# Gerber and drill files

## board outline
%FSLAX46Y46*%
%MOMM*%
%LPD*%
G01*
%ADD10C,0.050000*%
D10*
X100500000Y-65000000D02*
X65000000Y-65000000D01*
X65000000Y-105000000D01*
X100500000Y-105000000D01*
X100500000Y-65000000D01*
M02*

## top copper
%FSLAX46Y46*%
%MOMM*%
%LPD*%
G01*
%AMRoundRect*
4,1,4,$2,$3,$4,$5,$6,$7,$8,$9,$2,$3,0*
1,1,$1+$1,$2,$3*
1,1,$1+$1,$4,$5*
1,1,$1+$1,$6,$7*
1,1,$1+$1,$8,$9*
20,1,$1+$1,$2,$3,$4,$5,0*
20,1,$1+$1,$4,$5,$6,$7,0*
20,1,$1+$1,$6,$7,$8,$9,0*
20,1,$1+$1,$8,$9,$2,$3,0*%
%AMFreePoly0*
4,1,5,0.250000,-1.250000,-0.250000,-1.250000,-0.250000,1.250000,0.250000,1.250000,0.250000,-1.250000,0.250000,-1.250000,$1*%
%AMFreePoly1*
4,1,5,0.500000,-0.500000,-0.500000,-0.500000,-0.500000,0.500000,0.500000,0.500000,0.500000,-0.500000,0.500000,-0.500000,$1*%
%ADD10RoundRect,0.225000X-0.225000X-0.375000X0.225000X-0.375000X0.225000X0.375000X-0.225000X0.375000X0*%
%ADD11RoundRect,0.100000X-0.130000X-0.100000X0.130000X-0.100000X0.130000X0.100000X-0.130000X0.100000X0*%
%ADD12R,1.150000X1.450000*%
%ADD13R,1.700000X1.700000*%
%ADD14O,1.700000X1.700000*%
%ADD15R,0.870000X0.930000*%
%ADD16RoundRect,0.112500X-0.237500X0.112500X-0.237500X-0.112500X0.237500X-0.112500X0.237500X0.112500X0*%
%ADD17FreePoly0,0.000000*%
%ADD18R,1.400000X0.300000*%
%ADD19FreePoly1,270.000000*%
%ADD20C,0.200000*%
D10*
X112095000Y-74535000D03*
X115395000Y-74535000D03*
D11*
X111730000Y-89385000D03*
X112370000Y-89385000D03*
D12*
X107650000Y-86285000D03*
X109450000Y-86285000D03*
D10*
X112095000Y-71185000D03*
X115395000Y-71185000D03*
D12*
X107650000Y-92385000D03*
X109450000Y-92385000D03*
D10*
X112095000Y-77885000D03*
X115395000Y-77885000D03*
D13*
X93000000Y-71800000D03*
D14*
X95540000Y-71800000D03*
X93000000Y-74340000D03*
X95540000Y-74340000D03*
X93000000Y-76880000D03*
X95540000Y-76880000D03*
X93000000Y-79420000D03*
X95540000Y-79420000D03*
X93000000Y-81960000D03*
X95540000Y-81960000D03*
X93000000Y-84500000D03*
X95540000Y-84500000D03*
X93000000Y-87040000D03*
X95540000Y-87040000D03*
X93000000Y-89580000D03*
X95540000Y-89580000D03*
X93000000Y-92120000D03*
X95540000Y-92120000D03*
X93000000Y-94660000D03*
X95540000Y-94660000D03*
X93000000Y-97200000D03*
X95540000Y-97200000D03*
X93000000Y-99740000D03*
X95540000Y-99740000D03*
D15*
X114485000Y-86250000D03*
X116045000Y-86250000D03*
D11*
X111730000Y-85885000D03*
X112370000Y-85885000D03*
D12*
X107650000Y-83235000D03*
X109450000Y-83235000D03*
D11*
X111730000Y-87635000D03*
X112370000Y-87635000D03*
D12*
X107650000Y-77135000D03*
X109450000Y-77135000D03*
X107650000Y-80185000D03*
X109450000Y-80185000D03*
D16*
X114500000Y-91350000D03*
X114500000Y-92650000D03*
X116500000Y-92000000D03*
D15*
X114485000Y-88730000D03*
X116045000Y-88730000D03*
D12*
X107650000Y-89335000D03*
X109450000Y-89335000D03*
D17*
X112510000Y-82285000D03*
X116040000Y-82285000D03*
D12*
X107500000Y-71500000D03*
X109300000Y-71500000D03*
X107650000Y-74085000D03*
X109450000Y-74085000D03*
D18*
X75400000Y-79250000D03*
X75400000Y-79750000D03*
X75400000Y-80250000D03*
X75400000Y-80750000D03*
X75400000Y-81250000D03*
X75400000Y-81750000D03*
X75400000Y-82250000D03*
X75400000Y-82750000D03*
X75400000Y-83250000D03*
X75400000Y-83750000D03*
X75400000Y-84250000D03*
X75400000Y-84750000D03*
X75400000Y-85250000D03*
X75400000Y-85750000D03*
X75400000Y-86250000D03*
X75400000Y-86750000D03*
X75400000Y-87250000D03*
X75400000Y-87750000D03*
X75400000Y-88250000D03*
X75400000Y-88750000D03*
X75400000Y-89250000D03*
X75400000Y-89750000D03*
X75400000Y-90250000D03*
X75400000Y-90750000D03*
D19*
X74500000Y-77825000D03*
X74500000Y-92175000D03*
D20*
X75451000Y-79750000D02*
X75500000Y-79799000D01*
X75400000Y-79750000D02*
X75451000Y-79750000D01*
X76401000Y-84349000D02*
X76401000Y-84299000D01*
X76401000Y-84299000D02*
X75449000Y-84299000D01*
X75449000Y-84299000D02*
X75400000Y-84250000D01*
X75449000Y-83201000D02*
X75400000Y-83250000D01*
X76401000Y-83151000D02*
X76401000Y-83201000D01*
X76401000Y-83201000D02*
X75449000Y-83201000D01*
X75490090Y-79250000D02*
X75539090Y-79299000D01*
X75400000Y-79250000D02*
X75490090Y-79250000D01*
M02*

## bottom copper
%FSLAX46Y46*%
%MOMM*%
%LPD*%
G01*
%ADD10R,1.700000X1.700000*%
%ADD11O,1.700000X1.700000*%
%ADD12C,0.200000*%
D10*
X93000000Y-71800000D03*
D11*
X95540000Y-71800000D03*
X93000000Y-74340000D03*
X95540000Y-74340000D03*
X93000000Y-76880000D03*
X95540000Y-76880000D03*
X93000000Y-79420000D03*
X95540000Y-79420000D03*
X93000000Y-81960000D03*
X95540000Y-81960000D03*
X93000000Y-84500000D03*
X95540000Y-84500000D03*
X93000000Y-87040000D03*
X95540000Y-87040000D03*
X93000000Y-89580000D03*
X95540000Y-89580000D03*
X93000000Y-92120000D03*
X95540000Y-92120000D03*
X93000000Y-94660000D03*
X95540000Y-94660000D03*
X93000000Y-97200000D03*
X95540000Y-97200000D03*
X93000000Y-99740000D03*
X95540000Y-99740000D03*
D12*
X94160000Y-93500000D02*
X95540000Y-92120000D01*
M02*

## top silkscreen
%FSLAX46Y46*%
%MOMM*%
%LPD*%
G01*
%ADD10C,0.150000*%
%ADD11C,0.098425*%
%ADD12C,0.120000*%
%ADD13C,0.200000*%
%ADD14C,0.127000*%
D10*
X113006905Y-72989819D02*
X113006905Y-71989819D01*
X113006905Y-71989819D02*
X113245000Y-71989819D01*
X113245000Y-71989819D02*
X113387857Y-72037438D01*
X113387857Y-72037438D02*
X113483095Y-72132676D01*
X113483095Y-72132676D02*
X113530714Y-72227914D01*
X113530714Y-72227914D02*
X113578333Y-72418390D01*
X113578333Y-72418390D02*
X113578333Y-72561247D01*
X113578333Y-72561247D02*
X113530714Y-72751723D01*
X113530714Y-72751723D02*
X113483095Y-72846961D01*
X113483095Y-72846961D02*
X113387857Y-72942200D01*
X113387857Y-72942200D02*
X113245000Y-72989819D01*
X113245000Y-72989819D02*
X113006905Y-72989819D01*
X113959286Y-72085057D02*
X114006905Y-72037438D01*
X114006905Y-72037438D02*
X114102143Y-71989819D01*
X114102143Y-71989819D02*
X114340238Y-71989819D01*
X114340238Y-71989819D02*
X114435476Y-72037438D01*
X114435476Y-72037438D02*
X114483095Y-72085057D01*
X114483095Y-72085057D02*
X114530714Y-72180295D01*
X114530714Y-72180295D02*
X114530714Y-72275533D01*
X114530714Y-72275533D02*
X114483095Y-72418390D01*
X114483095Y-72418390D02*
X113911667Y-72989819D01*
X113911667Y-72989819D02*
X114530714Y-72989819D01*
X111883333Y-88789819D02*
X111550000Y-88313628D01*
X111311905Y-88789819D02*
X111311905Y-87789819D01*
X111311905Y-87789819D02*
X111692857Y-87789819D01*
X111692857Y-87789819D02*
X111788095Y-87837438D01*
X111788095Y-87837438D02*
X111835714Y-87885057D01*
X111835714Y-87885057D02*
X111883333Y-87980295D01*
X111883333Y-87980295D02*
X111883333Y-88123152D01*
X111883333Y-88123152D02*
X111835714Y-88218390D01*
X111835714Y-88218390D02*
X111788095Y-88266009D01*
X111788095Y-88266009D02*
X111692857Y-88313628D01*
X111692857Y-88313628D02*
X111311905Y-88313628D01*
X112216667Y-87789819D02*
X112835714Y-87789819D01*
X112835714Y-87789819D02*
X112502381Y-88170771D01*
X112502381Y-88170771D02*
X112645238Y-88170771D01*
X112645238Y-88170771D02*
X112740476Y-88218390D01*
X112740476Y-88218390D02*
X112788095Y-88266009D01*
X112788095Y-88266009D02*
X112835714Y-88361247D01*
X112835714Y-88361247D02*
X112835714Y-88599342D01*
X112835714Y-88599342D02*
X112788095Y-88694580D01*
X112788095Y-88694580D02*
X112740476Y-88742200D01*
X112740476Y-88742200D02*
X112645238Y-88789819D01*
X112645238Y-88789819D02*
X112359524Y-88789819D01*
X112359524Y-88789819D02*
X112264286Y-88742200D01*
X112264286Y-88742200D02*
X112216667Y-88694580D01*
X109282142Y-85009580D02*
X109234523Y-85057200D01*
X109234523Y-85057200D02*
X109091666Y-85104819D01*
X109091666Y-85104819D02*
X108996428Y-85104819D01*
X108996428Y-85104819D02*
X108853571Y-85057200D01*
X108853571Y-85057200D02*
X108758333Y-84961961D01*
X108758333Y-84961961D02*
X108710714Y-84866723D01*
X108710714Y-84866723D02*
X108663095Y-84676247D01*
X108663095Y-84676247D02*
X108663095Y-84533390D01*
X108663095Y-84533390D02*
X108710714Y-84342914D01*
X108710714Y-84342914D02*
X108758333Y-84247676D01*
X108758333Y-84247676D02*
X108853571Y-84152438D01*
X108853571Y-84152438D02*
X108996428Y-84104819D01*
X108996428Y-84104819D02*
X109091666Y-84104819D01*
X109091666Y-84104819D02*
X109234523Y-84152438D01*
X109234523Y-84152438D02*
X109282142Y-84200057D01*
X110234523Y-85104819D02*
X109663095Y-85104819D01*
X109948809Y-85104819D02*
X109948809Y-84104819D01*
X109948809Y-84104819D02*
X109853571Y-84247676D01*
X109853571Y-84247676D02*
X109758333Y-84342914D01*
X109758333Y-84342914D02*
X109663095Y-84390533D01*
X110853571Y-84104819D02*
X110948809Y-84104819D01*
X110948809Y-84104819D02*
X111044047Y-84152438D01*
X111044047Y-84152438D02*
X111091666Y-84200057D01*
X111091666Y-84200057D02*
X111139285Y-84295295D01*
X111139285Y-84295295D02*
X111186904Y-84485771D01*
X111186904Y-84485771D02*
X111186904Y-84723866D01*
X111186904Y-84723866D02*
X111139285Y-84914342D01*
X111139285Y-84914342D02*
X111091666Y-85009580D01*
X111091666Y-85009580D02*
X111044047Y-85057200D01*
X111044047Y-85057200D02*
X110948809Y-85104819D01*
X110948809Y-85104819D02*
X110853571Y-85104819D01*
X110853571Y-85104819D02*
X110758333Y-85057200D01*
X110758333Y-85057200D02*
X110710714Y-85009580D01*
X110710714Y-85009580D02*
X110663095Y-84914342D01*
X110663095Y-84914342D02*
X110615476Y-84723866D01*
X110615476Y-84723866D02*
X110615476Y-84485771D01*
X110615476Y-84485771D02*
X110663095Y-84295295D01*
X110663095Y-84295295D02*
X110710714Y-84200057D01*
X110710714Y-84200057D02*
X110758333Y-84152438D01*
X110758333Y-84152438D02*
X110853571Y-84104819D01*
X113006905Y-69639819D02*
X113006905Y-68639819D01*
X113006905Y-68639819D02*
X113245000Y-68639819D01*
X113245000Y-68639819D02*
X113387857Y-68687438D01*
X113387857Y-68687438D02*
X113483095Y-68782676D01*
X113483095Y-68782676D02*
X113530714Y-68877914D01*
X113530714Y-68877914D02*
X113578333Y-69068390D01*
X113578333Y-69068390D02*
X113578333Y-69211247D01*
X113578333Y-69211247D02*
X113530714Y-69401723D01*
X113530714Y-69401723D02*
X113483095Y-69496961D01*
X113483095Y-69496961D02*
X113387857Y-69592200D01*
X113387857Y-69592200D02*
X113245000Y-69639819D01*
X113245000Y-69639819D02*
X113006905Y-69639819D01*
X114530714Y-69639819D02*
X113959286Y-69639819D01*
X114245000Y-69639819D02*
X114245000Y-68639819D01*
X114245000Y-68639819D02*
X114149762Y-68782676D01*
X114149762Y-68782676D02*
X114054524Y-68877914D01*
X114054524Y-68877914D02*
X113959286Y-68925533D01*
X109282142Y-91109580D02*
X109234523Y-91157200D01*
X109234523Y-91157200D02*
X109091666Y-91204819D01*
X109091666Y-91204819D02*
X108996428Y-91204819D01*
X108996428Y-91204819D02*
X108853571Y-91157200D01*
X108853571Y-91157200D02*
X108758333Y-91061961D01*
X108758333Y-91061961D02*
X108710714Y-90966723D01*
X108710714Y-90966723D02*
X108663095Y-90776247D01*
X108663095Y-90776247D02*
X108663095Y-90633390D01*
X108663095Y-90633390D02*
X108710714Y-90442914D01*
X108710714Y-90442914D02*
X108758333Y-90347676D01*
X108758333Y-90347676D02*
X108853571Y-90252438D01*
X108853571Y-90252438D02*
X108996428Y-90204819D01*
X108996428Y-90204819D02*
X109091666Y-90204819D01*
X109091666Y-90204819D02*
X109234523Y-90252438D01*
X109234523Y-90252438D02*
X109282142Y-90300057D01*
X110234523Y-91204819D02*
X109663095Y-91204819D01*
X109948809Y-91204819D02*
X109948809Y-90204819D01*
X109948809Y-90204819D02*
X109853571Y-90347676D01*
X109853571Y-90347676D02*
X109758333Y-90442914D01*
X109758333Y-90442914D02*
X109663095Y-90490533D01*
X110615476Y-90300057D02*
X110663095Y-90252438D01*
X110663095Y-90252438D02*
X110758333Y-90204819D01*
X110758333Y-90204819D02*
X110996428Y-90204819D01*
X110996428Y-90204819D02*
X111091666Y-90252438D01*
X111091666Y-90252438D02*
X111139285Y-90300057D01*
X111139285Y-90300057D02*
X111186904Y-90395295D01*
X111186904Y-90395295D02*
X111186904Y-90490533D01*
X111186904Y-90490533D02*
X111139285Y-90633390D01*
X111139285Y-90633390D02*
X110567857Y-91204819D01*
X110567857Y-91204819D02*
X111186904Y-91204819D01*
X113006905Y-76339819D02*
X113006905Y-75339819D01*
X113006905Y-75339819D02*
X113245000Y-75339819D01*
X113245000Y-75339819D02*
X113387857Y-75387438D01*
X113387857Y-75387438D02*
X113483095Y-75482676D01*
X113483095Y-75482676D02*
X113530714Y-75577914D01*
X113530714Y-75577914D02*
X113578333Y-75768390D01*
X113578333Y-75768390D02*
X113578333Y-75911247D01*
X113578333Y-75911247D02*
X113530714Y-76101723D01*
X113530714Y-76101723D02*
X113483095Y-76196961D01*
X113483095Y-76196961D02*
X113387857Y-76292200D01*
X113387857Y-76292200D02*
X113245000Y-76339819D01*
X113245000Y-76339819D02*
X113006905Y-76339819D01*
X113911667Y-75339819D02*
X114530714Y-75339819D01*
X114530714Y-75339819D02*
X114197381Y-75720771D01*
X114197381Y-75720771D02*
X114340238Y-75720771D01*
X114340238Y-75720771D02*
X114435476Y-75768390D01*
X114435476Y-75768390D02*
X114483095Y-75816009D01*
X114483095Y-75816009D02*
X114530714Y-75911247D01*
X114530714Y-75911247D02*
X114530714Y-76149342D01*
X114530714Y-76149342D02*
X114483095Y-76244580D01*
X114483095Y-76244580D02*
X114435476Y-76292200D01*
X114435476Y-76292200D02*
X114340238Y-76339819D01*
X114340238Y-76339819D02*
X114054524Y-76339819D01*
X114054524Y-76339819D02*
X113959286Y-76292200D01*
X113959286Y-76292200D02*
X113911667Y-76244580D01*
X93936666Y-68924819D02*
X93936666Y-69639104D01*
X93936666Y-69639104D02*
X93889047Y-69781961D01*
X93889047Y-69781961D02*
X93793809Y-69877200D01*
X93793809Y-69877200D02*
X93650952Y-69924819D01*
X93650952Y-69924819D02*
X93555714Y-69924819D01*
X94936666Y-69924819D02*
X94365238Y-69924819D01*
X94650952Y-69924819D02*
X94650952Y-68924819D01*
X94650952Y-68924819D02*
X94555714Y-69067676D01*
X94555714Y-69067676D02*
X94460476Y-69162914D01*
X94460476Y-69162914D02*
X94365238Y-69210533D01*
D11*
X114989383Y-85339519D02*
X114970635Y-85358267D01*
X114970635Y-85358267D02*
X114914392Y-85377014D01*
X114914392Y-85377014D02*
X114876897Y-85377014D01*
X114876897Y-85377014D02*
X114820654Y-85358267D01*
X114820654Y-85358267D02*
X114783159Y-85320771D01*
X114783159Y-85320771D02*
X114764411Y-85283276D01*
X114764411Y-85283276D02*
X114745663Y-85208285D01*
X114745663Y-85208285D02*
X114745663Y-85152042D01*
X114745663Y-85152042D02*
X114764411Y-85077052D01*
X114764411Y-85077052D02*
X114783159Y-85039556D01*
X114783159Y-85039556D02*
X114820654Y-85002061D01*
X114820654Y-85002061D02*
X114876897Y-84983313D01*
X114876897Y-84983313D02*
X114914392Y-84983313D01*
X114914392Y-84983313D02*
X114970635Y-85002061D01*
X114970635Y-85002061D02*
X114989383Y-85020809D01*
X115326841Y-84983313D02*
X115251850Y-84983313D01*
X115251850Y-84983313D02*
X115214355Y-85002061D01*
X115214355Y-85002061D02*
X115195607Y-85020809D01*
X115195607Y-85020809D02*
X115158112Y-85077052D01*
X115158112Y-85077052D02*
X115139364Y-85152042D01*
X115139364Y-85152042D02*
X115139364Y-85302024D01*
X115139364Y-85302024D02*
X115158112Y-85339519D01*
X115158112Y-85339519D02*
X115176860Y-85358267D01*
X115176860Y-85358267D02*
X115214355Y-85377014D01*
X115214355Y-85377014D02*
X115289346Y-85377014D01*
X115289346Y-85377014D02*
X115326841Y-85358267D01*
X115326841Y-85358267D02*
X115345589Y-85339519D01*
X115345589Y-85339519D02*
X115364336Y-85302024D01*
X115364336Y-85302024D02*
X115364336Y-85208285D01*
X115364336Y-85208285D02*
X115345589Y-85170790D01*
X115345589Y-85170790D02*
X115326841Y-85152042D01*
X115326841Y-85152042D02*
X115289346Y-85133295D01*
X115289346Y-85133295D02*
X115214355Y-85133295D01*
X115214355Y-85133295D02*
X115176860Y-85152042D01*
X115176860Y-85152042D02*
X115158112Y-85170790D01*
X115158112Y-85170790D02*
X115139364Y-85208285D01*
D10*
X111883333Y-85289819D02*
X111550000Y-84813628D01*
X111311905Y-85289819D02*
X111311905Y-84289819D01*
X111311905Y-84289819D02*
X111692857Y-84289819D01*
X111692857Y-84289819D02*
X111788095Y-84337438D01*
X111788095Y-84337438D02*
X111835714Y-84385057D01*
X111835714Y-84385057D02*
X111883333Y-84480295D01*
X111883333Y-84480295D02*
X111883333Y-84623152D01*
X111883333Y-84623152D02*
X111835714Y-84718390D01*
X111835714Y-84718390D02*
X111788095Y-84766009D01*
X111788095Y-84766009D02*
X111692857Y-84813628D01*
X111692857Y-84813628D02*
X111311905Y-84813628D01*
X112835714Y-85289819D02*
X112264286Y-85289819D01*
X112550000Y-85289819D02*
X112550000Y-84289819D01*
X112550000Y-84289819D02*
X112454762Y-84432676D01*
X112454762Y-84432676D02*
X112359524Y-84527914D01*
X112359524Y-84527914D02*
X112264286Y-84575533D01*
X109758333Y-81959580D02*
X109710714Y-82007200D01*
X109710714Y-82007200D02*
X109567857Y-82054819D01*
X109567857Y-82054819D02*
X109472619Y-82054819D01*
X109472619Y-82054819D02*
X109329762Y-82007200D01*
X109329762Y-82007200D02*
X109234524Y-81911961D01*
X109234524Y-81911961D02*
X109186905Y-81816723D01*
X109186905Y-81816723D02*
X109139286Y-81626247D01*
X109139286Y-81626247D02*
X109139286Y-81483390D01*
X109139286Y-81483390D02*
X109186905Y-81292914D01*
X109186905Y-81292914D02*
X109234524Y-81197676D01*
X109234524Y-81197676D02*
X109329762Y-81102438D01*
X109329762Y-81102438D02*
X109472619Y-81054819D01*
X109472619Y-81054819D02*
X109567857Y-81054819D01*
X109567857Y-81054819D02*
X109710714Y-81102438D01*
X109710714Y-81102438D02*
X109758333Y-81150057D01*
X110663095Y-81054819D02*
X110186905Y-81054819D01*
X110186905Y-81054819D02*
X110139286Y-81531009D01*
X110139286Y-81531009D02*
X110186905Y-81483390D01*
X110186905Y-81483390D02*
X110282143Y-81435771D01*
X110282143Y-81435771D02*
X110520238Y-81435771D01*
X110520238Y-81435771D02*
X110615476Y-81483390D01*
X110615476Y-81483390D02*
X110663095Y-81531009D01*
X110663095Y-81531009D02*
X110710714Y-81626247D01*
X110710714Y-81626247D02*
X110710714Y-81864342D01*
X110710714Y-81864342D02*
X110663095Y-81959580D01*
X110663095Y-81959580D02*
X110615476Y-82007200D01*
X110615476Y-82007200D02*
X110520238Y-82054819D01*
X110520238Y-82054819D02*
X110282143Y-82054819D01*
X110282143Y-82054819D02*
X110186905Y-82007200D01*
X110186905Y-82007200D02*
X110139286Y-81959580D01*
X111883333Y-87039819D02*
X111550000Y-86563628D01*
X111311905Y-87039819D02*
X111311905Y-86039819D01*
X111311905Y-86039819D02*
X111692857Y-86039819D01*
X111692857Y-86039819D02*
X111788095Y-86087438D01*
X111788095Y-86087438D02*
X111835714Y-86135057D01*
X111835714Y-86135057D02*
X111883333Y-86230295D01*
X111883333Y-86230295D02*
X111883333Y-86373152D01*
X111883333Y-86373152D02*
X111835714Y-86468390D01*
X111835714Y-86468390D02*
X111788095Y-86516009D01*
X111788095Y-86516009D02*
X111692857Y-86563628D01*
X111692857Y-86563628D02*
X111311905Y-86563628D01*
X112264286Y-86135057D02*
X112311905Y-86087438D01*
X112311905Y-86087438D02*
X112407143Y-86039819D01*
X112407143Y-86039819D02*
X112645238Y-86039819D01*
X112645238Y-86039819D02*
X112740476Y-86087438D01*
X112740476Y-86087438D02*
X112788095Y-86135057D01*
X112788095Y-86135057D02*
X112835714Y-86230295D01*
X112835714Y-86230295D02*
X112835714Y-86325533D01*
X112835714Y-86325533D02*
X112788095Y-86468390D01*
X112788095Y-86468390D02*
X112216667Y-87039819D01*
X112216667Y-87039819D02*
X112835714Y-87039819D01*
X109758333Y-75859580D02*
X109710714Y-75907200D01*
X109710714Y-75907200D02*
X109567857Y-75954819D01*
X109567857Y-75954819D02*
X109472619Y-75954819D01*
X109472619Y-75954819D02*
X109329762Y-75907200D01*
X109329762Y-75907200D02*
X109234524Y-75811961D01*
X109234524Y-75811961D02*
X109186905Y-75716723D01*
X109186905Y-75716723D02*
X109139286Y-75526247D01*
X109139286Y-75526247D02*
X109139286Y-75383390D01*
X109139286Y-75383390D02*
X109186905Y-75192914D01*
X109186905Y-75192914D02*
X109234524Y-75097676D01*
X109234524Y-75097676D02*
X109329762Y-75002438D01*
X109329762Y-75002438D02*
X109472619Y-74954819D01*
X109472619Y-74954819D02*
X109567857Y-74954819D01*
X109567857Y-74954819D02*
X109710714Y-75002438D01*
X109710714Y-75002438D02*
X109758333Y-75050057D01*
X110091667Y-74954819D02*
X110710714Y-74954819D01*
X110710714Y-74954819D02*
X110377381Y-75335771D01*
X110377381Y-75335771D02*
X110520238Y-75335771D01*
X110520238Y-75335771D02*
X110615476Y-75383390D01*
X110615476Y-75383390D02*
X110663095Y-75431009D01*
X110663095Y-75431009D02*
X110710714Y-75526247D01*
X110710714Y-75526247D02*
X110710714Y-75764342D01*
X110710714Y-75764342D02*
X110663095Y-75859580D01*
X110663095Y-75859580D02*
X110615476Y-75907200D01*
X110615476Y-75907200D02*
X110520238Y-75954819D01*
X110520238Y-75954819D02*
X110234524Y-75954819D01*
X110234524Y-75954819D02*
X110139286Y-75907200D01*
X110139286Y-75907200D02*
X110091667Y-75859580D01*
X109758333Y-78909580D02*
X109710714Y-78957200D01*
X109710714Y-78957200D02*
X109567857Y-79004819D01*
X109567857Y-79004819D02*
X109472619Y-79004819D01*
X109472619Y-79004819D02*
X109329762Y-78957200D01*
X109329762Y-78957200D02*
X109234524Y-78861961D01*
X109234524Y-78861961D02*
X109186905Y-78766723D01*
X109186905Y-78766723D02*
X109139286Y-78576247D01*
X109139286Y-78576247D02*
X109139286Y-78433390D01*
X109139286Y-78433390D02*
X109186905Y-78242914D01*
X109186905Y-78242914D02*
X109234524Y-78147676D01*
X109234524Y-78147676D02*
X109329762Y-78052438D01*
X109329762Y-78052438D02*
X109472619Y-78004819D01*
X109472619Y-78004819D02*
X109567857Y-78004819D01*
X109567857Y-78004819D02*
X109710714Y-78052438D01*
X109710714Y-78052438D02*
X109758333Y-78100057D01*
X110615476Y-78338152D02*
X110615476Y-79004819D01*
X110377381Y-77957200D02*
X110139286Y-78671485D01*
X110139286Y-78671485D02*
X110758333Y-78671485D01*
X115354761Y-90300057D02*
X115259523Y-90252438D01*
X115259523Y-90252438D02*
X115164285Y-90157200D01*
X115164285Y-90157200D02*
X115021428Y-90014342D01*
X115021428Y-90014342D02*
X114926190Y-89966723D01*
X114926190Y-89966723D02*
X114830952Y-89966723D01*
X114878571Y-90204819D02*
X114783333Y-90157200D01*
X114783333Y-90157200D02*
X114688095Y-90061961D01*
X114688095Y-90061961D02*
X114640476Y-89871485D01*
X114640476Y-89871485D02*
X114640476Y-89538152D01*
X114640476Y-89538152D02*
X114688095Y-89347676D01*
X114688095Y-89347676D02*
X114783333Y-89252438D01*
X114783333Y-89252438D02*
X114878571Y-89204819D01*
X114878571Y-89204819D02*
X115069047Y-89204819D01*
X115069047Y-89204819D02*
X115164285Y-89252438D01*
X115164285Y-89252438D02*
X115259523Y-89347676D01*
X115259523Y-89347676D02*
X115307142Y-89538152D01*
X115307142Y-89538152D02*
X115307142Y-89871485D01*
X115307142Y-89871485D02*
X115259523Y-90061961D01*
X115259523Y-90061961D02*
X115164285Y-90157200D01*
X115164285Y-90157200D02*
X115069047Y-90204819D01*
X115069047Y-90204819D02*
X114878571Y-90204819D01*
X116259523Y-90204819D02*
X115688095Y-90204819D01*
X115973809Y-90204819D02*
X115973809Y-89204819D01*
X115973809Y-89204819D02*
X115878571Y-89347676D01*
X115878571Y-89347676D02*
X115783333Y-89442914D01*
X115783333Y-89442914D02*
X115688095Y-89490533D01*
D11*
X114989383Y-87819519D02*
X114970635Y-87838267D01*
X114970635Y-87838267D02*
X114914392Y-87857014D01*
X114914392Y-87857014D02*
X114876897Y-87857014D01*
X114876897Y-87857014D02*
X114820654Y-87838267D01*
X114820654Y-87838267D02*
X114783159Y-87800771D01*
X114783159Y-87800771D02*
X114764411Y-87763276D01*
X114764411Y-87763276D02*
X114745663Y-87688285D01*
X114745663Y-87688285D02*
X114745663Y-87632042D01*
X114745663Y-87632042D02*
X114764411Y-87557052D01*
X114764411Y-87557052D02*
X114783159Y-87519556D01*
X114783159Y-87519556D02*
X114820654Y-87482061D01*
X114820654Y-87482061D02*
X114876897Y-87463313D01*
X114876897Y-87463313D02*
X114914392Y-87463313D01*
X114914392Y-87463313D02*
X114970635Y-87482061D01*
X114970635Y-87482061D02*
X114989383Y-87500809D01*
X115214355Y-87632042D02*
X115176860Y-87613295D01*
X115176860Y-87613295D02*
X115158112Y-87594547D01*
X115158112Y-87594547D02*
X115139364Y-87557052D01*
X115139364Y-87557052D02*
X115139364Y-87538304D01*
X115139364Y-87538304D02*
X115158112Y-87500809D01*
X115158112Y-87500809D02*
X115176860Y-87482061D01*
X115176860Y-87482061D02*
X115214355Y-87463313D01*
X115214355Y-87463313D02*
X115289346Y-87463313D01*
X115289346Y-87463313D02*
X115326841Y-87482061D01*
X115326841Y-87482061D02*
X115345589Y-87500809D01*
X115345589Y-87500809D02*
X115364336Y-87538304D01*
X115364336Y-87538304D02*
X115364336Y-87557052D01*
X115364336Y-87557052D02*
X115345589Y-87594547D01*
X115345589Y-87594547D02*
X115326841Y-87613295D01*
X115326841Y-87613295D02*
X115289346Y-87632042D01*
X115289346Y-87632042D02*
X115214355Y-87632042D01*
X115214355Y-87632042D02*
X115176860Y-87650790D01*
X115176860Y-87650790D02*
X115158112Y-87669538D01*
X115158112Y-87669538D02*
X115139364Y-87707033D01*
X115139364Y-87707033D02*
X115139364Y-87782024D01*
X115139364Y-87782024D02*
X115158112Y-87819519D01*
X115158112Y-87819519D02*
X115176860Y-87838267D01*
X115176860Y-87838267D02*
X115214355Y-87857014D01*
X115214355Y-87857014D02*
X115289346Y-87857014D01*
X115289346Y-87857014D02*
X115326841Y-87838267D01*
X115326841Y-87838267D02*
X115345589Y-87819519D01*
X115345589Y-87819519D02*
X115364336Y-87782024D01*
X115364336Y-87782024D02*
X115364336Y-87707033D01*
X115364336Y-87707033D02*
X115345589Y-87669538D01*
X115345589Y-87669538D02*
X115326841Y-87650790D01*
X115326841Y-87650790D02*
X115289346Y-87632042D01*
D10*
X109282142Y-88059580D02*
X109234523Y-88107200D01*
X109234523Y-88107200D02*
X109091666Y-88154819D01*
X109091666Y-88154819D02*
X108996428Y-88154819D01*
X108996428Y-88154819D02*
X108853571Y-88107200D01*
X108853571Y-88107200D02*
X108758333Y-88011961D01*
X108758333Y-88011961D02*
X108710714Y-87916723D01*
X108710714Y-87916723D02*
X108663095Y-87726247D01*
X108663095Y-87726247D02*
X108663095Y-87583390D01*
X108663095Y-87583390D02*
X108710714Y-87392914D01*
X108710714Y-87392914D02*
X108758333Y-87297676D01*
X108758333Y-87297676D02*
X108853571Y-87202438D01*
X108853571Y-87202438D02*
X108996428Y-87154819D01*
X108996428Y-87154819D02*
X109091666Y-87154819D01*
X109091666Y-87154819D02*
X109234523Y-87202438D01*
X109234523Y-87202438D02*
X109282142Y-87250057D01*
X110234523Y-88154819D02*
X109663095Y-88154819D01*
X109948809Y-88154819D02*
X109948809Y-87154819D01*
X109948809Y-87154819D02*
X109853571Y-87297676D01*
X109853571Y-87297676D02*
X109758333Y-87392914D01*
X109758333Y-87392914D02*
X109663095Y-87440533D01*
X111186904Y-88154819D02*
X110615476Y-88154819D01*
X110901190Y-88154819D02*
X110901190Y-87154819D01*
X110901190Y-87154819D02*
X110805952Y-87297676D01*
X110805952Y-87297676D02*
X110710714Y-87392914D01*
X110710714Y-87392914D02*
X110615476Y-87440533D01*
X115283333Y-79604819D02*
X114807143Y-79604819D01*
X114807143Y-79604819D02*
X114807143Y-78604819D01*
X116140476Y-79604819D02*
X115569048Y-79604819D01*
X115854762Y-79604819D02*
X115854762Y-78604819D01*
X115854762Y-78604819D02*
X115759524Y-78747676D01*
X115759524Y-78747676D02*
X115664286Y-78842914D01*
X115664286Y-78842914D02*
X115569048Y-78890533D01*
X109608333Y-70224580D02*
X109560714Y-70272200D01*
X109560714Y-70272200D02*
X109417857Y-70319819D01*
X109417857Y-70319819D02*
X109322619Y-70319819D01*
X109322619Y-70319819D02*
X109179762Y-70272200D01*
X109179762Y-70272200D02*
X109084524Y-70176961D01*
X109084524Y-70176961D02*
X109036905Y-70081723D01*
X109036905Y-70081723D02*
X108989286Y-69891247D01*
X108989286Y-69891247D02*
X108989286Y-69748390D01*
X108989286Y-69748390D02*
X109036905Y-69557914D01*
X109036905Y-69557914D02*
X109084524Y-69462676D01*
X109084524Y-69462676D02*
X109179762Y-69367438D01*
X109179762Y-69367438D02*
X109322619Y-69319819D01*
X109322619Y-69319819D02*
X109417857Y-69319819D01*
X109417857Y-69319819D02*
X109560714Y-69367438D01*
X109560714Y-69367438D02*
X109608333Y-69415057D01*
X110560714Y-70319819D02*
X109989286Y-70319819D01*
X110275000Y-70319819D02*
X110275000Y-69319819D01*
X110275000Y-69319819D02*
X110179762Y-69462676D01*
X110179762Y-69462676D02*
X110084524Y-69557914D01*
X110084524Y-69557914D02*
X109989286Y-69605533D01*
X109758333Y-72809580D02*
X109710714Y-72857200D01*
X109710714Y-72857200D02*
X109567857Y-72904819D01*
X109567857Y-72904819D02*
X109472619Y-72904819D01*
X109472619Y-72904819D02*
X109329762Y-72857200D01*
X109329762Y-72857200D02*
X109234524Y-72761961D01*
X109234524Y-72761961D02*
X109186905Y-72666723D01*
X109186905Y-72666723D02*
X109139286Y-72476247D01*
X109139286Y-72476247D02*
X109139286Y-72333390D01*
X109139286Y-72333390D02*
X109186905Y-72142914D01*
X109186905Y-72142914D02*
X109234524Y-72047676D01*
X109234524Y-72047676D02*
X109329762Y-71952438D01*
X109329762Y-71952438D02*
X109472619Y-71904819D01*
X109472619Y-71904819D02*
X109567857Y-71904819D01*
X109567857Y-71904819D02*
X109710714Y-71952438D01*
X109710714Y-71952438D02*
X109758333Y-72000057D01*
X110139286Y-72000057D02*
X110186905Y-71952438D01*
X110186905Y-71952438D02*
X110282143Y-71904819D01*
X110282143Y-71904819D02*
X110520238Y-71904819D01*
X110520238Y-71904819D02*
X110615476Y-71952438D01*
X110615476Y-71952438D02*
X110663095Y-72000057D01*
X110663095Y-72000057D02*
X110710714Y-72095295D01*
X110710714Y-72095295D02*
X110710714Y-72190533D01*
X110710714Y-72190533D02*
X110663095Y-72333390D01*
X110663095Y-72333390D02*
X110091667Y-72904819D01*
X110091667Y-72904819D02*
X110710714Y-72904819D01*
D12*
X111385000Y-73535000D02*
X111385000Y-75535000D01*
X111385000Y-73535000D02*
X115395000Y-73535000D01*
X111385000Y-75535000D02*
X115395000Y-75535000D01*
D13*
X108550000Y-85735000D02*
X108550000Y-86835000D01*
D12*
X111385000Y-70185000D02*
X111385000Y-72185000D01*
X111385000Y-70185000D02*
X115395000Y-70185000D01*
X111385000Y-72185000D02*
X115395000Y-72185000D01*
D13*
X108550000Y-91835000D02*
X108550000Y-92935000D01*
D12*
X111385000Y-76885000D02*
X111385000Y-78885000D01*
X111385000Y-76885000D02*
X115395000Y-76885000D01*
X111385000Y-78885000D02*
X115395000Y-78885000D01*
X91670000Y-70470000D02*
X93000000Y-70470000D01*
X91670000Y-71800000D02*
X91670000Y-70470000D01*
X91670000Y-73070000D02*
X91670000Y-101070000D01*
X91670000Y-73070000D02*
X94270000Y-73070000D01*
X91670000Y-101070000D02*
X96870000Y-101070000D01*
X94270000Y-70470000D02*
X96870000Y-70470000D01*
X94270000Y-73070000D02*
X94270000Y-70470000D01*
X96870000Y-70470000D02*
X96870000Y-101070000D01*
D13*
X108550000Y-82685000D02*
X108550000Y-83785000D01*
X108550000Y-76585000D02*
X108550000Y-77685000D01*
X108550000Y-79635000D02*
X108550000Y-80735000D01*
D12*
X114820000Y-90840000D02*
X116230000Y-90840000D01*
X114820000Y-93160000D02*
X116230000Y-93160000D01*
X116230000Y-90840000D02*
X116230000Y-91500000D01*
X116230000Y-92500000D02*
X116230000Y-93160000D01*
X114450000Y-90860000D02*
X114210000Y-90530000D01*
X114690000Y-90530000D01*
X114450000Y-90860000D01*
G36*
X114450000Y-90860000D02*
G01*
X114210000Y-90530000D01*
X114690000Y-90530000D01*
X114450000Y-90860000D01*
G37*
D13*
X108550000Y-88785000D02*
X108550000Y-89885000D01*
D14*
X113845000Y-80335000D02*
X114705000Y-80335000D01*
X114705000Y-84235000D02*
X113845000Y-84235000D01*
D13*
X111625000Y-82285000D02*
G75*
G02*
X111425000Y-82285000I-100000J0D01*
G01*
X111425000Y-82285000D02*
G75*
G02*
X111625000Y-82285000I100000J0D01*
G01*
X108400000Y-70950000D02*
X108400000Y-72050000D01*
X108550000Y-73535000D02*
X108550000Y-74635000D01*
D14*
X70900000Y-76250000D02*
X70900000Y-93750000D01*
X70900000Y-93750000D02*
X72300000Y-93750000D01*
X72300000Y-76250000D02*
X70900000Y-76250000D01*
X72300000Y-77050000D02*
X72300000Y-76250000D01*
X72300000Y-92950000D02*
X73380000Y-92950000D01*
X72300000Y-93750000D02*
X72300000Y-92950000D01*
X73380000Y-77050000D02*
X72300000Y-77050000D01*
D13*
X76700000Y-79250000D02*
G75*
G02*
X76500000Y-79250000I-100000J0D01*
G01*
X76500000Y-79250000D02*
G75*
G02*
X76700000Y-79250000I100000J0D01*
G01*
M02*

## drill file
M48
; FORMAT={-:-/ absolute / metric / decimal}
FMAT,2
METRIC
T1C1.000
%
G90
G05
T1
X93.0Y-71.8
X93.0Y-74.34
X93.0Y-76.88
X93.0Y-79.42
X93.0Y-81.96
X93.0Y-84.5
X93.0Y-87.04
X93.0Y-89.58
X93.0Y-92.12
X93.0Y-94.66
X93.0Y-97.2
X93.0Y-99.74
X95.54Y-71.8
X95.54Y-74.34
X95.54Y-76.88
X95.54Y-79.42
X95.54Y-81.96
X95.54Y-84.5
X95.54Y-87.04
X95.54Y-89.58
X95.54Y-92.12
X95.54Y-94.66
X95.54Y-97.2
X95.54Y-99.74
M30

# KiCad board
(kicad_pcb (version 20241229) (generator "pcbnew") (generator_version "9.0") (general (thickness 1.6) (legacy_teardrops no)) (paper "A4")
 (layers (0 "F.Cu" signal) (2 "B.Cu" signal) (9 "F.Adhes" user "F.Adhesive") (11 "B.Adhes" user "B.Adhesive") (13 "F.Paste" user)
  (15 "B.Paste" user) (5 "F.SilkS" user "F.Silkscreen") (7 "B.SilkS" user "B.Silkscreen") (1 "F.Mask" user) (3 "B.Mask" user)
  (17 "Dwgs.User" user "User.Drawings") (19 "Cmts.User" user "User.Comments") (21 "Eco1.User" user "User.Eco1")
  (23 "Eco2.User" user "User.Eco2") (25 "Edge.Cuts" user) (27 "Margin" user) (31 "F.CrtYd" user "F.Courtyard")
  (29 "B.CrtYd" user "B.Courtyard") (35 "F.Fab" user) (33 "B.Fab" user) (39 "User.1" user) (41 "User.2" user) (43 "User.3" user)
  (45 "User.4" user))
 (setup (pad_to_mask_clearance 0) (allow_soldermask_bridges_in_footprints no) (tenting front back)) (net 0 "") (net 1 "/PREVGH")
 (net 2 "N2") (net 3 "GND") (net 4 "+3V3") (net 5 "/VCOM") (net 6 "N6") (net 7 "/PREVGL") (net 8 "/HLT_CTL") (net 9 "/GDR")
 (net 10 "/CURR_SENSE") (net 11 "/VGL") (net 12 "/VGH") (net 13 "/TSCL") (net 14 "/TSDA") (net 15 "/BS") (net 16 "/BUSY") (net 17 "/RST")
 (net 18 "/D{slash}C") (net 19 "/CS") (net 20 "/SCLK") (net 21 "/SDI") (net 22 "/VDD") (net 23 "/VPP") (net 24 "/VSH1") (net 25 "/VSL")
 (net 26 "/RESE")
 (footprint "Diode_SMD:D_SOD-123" (layer "F.Cu") (at 113.745 74.535)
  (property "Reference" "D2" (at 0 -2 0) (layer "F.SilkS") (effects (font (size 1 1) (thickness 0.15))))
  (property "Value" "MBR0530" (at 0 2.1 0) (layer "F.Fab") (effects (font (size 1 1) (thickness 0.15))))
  (fp_line (start -2.36 -1) (end -2.36 1) (stroke (width 0.12) (type solid)) (layer "F.SilkS"))
  (fp_line (start -2.36 -1) (end 1.65 -1) (stroke (width 0.12) (type solid)) (layer "F.SilkS"))
  (fp_line (start -2.36 1) (end 1.65 1) (stroke (width 0.12) (type solid)) (layer "F.SilkS"))
  (pad "1" smd roundrect (at -1.65 0) (size 0.9 1.2) (layers "F.Cu" "F.Mask" "F.Paste") (roundrect_rratio 0.25) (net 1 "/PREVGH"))
  (pad "2" smd roundrect (at 1.65 0) (size 0.9 1.2) (layers "F.Cu" "F.Mask" "F.Paste") (roundrect_rratio 0.25) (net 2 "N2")))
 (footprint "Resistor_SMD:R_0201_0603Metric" (layer "F.Cu") (at 112.05 89.385)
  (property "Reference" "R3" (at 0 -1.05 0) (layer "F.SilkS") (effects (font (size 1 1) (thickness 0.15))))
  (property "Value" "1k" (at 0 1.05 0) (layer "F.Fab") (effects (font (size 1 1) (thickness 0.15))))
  (pad "" smd roundrect (at -0.345 0) (size 0.318 0.36) (layers "F.Paste") (roundrect_rratio 0.25))
  (pad "" smd roundrect (at 0.345 0) (size 0.318 0.36) (layers "F.Paste") (roundrect_rratio 0.25))
  (pad "1" smd roundrect (at -0.32 0) (size 0.46 0.4) (layers "F.Cu" "F.Mask") (roundrect_rratio 0.25) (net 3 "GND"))
  (pad "2" smd roundrect (at 0.32 0) (size 0.46 0.4) (layers "F.Cu" "F.Mask") (roundrect_rratio 0.25) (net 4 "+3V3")))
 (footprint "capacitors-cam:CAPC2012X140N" (layer "F.Cu") (at 108.55 86.285)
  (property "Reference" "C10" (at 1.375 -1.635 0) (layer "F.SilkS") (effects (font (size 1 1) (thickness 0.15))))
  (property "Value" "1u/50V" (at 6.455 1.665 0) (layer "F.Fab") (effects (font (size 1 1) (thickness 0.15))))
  (fp_line (start 0 -0.55) (end 0 0.55) (stroke (width 0.2) (type solid)) (layer "F.SilkS"))
  (pad "1" smd rect (at -0.9 0) (size 1.15 1.45) (layers "F.Cu" "F.Mask" "F.Paste") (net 3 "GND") (solder_mask_margin 0.102))
  (pad "2" smd rect (at 0.9 0) (size 1.15 1.45) (layers "F.Cu" "F.Mask" "F.Paste") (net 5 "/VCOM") (solder_mask_margin 0.102)))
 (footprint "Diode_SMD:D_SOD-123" (layer "F.Cu") (at 113.745 71.185)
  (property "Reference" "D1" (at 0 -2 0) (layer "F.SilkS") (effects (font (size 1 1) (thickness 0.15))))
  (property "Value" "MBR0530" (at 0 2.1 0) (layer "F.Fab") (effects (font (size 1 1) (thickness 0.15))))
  (fp_line (start -2.36 -1) (end -2.36 1) (stroke (width 0.12) (type solid)) (layer "F.SilkS"))
  (fp_line (start -2.36 -1) (end 1.65 -1) (stroke (width 0.12) (type solid)) (layer "F.SilkS"))
  (fp_line (start -2.36 1) (end 1.65 1) (stroke (width 0.12) (type solid)) (layer "F.SilkS"))
  (pad "1" smd roundrect (at -1.65 0) (size 0.9 1.2) (layers "F.Cu" "F.Mask" "F.Paste") (roundrect_rratio 0.25) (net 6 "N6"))
  (pad "2" smd roundrect (at 1.65 0) (size 0.9 1.2) (layers "F.Cu" "F.Mask" "F.Paste") (roundrect_rratio 0.25) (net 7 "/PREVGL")))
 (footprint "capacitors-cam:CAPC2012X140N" (layer "F.Cu") (at 108.55 92.385)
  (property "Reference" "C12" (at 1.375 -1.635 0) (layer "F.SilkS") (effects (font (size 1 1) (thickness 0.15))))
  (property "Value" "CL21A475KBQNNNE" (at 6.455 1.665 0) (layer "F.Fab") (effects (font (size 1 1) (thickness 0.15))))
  (fp_line (start 0 -0.55) (end 0 0.55) (stroke (width 0.2) (type solid)) (layer "F.SilkS"))
  (pad "1" smd rect (at -0.9 0) (size 1.15 1.45) (layers "F.Cu" "F.Mask" "F.Paste") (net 3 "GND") (solder_mask_margin 0.102))
  (pad "2" smd rect (at 0.9 0) (size 1.15 1.45) (layers "F.Cu" "F.Mask" "F.Paste") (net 4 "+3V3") (solder_mask_margin 0.102)))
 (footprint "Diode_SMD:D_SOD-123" (layer "F.Cu") (at 113.745 77.885)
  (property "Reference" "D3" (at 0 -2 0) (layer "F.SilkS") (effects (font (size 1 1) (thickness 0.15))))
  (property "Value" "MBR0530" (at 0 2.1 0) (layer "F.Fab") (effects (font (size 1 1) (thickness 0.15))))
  (fp_line (start -2.36 -1) (end -2.36 1) (stroke (width 0.12) (type solid)) (layer "F.SilkS"))
  (fp_line (start -2.36 -1) (end 1.65 -1) (stroke (width 0.12) (type solid)) (layer "F.SilkS"))
  (fp_line (start -2.36 1) (end 1.65 1) (stroke (width 0.12) (type solid)) (layer "F.SilkS"))
  (pad "1" smd roundrect (at -1.65 0) (size 0.9 1.2) (layers "F.Cu" "F.Mask" "F.Paste") (roundrect_rratio 0.25) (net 3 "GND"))
  (pad "2" smd roundrect (at 1.65 0) (size 0.9 1.2) (layers "F.Cu" "F.Mask" "F.Paste") (roundrect_rratio 0.25) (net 6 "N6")))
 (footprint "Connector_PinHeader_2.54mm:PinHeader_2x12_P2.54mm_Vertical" (layer "F.Cu") (at 93 71.8)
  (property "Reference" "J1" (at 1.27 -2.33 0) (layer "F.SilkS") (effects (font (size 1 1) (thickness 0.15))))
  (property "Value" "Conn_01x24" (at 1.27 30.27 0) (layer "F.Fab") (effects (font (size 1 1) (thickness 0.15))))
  (fp_line (start -1.33 -1.33) (end 0 -1.33) (stroke (width 0.12) (type solid)) (layer "F.SilkS"))
  (fp_line (start -1.33 0) (end -1.33 -1.33) (stroke (width 0.12) (type solid)) (layer "F.SilkS"))
  (fp_line (start -1.33 1.27) (end -1.33 29.27) (stroke (width 0.12) (type solid)) (layer "F.SilkS"))
  (fp_line (start -1.33 1.27) (end 1.27 1.27) (stroke (width 0.12) (type solid)) (layer "F.SilkS"))
  (fp_line (start -1.33 29.27) (end 3.87 29.27) (stroke (width 0.12) (type solid)) (layer "F.SilkS"))
  (fp_line (start 1.27 -1.33) (end 3.87 -1.33) (stroke (width 0.12) (type solid)) (layer "F.SilkS"))
  (fp_line (start 1.27 1.27) (end 1.27 -1.33) (stroke (width 0.12) (type solid)) (layer "F.SilkS"))
  (fp_line (start 3.87 -1.33) (end 3.87 29.27) (stroke (width 0.12) (type solid)) (layer "F.SilkS"))
  (pad "1" thru_hole rect (at 0 0) (size 1.7 1.7) (drill 1) (layers "*.Cu" "*.Mask") (remove_unused_layers no) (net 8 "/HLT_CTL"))
  (pad "2" thru_hole oval (at 2.54 0) (size 1.7 1.7) (drill 1) (layers "*.Cu" "*.Mask") (remove_unused_layers no) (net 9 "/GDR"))
  (pad "3" thru_hole oval (at 0 2.54) (size 1.7 1.7) (drill 1) (layers "*.Cu" "*.Mask") (remove_unused_layers no) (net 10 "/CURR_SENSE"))
  (pad "4" thru_hole oval (at 2.54 2.54) (size 1.7 1.7) (drill 1) (layers "*.Cu" "*.Mask") (remove_unused_layers no) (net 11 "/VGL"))
  (pad "5" thru_hole oval (at 0 5.08) (size 1.7 1.7) (drill 1) (layers "*.Cu" "*.Mask") (remove_unused_layers no) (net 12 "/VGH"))
  (pad "6" thru_hole oval (at 2.54 5.08) (size 1.7 1.7) (drill 1) (layers "*.Cu" "*.Mask") (remove_unused_layers no) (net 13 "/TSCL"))
  (pad "7" thru_hole oval (at 0 7.62) (size 1.7 1.7) (drill 1) (layers "*.Cu" "*.Mask") (remove_unused_layers no) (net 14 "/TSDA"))
  (pad "8" thru_hole oval (at 2.54 7.62) (size 1.7 1.7) (drill 1) (layers "*.Cu" "*.Mask") (remove_unused_layers no) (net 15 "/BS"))
  (pad "9" thru_hole oval (at 0 10.16) (size 1.7 1.7) (drill 1) (layers "*.Cu" "*.Mask") (remove_unused_layers no) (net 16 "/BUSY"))
  (pad "10" thru_hole oval (at 2.54 10.16) (size 1.7 1.7) (drill 1) (layers "*.Cu" "*.Mask") (remove_unused_layers no) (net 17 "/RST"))
  (pad "11" thru_hole oval (at 0 12.7) (size 1.7 1.7) (drill 1) (layers "*.Cu" "*.Mask") (remove_unused_layers no) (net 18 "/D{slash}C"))
  (pad "12" thru_hole oval (at 2.54 12.7) (size 1.7 1.7) (drill 1) (layers "*.Cu" "*.Mask") (remove_unused_layers no) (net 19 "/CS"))
  (pad "13" thru_hole oval (at 0 15.24) (size 1.7 1.7) (drill 1) (layers "*.Cu" "*.Mask") (remove_unused_layers no) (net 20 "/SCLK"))
  (pad "14" thru_hole oval (at 2.54 15.24) (size 1.7 1.7) (drill 1) (layers "*.Cu" "*.Mask") (remove_unused_layers no) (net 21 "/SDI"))
  (pad "15" thru_hole oval (at 0 17.78) (size 1.7 1.7) (drill 1) (layers "*.Cu" "*.Mask") (remove_unused_layers no) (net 4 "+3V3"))
  (pad "16" thru_hole oval (at 2.54 17.78) (size 1.7 1.7) (drill 1) (layers "*.Cu" "*.Mask") (remove_unused_layers no) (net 4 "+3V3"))
  (pad "17" thru_hole oval (at 0 20.32) (size 1.7 1.7) (drill 1) (layers "*.Cu" "*.Mask") (remove_unused_layers no) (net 3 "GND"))
  (pad "18" thru_hole oval (at 2.54 20.32) (size 1.7 1.7) (drill 1) (layers "*.Cu" "*.Mask") (remove_unused_layers no) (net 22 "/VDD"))
  (pad "19" thru_hole oval (at 0 22.86) (size 1.7 1.7) (drill 1) (layers "*.Cu" "*.Mask") (remove_unused_layers no) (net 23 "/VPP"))
  (pad "20" thru_hole oval (at 2.54 22.86) (size 1.7 1.7) (drill 1) (layers "*.Cu" "*.Mask") (remove_unused_layers no) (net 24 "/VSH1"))
  (pad "21" thru_hole oval (at 0 25.4) (size 1.7 1.7) (drill 1) (layers "*.Cu" "*.Mask") (remove_unused_layers no) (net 1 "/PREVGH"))
  (pad "22" thru_hole oval (at 2.54 25.4) (size 1.7 1.7) (drill 1) (layers "*.Cu" "*.Mask") (remove_unused_layers no) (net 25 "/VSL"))
  (pad "23" thru_hole oval (at 0 27.94) (size 1.7 1.7) (drill 1) (layers "*.Cu" "*.Mask") (remove_unused_layers no) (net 7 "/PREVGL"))
  (pad "24" thru_hole oval (at 2.54 27.94) (size 1.7 1.7) (drill 1) (layers "*.Cu" "*.Mask") (remove_unused_layers no) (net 5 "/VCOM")))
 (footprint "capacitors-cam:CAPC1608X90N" (layer "F.Cu") (at 115.265 86.25)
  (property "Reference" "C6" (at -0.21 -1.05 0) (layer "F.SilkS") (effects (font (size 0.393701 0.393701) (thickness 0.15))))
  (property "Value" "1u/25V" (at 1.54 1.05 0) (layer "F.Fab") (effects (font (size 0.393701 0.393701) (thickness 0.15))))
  (pad "1" smd rect (at -0.78 0) (size 0.87 0.93) (layers "F.Cu" "F.Mask" "F.Paste") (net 3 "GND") (solder_mask_margin 0.102))
  (pad "2" smd rect (at 0.78 0) (size 0.87 0.93) (layers "F.Cu" "F.Mask" "F.Paste") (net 24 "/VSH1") (solder_mask_margin 0.102)))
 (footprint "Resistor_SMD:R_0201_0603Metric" (layer "F.Cu") (at 112.05 85.885)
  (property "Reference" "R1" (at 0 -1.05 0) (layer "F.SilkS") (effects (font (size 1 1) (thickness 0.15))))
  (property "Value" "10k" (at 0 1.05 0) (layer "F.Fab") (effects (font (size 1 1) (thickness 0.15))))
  (pad "" smd roundrect (at -0.345 0) (size 0.318 0.36) (layers "F.Paste") (roundrect_rratio 0.25))
  (pad "" smd roundrect (at 0.345 0) (size 0.318 0.36) (layers "F.Paste") (roundrect_rratio 0.25))
  (pad "1" smd roundrect (at -0.32 0) (size 0.46 0.4) (layers "F.Cu" "F.Mask") (roundrect_rratio 0.25) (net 3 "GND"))
  (pad "2" smd roundrect (at 0.32 0) (size 0.46 0.4) (layers "F.Cu" "F.Mask") (roundrect_rratio 0.25) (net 9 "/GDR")))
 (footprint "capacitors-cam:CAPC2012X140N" (layer "F.Cu") (at 108.55 83.235)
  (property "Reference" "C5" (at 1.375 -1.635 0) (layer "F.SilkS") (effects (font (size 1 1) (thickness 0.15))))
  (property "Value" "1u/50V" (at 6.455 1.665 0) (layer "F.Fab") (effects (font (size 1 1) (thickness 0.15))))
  (fp_line (start 0 -0.55) (end 0 0.55) (stroke (width 0.2) (type solid)) (layer "F.SilkS"))
  (pad "1" smd rect (at -0.9 0) (size 1.15 1.45) (layers "F.Cu" "F.Mask" "F.Paste") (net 3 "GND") (solder_mask_margin 0.102))
  (pad "2" smd rect (at 0.9 0) (size 1.15 1.45) (layers "F.Cu" "F.Mask" "F.Paste") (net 23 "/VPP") (solder_mask_margin 0.102)))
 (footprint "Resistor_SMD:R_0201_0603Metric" (layer "F.Cu") (at 112.05 87.635)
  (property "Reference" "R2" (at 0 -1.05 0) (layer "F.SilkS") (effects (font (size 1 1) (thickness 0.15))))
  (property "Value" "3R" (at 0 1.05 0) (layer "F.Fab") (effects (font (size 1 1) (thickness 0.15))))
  (pad "" smd roundrect (at -0.345 0) (size 0.318 0.36) (layers "F.Paste") (roundrect_rratio 0.25))
  (pad "" smd roundrect (at 0.345 0) (size 0.318 0.36) (layers "F.Paste") (roundrect_rratio 0.25))
  (pad "1" smd roundrect (at -0.32 0) (size 0.46 0.4) (layers "F.Cu" "F.Mask") (roundrect_rratio 0.25) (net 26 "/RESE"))
  (pad "2" smd roundrect (at 0.32 0) (size 0.46 0.4) (layers "F.Cu" "F.Mask") (roundrect_rratio 0.25) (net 3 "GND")))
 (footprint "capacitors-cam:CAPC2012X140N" (layer "F.Cu") (at 108.55 77.135)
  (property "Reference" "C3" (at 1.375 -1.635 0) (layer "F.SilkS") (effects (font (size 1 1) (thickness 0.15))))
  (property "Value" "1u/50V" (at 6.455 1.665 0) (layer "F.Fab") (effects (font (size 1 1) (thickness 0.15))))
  (fp_line (start 0 -0.55) (end 0 0.55) (stroke (width 0.2) (type solid)) (layer "F.SilkS"))
  (pad "1" smd rect (at -0.9 0) (size 1.15 1.45) (layers "F.Cu" "F.Mask" "F.Paste") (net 3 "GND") (solder_mask_margin 0.102))
  (pad "2" smd rect (at 0.9 0) (size 1.15 1.45) (layers "F.Cu" "F.Mask" "F.Paste") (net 4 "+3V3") (solder_mask_margin 0.102)))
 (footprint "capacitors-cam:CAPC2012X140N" (layer "F.Cu") (at 108.55 80.185)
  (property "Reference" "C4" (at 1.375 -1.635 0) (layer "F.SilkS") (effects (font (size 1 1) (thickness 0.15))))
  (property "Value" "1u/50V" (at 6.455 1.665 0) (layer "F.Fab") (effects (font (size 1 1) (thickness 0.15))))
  (fp_line (start 0 -0.55) (end 0 0.55) (stroke (width 0.2) (type solid)) (layer "F.SilkS"))
  (pad "1" smd rect (at -0.9 0) (size 1.15 1.45) (layers "F.Cu" "F.Mask" "F.Paste") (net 3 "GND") (solder_mask_margin 0.102))
  (pad "2" smd rect (at 0.9 0) (size 1.15 1.45) (layers "F.Cu" "F.Mask" "F.Paste") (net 22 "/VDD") (solder_mask_margin 0.102)))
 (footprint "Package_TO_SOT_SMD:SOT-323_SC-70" (layer "F.Cu") (at 115.5 92)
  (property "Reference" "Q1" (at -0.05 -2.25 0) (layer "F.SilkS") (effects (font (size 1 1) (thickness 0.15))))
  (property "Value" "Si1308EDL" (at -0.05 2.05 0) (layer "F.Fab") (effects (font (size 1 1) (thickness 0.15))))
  (fp_line (start -0.68 -1.16) (end 0.73 -1.16) (stroke (width 0.12) (type solid)) (layer "F.SilkS"))
  (fp_line (start -0.68 1.16) (end 0.73 1.16) (stroke (width 0.12) (type solid)) (layer "F.SilkS"))
  (fp_line (start 0.73 -1.16) (end 0.73 -0.5) (stroke (width 0.12) (type solid)) (layer "F.SilkS"))
  (fp_line (start 0.73 0.5) (end 0.73 1.16) (stroke (width 0.12) (type solid)) (layer "F.SilkS"))
  (fp_poly
   (pts (xy -1.05 -1.14) (xy -1.29 -1.47) (xy -0.81 -1.47) (xy -1.05 -1.14)) (stroke (width 0.12) (type solid)) (fill yes) (layer "F.SilkS"))
  (pad "1" smd roundrect (at -1 -0.65 270) (size 0.45 0.7) (layers "F.Cu" "F.Mask" "F.Paste") (roundrect_rratio 0.25) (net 9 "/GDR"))
  (pad "2" smd roundrect (at -1 0.65 270) (size 0.45 0.7) (layers "F.Cu" "F.Mask" "F.Paste") (roundrect_rratio 0.25) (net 2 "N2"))
  (pad "3" smd roundrect (at 1 0 270) (size 0.45 0.7) (layers "F.Cu" "F.Mask" "F.Paste") (roundrect_rratio 0.25) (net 26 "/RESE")))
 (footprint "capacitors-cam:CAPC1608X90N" (layer "F.Cu") (at 115.265 88.73)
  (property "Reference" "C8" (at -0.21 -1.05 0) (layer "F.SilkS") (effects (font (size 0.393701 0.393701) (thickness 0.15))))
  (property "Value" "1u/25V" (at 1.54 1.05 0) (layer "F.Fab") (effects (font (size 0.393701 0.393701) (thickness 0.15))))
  (pad "1" smd rect (at -0.78 0) (size 0.87 0.93) (layers "F.Cu" "F.Mask" "F.Paste") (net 3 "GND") (solder_mask_margin 0.102))
  (pad "2" smd rect (at 0.78 0) (size 0.87 0.93) (layers "F.Cu" "F.Mask" "F.Paste") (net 25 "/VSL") (solder_mask_margin 0.102)))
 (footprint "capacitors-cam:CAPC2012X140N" (layer "F.Cu") (at 108.55 89.335)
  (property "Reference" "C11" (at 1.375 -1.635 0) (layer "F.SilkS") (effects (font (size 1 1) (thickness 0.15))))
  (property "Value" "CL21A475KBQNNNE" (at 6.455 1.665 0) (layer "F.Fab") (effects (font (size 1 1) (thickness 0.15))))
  (fp_line (start 0 -0.55) (end 0 0.55) (stroke (width 0.2) (type solid)) (layer "F.SilkS"))
  (pad "1" smd rect (at -0.9 0) (size 1.15 1.45) (layers "F.Cu" "F.Mask" "F.Paste") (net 6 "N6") (solder_mask_margin 0.102))
  (pad "2" smd rect (at 0.9 0) (size 1.15 1.45) (layers "F.Cu" "F.Mask" "F.Paste") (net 2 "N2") (solder_mask_margin 0.102)))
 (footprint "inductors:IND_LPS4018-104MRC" (layer "F.Cu") (at 114.275 82.285)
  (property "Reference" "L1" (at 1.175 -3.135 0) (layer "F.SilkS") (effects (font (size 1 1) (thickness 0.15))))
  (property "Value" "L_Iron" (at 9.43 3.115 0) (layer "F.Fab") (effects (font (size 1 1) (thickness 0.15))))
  (fp_line (start -0.43 -1.95) (end 0.43 -1.95) (stroke (width 0.127) (type solid)) (layer "F.SilkS"))
  (fp_line (start 0.43 1.95) (end -0.43 1.95) (stroke (width 0.127) (type solid)) (layer "F.SilkS"))
  (fp_circle (center -2.75 0) (end -2.65 0) (stroke (width 0.2) (type solid)) (fill no) (layer "F.SilkS"))
  (pad "1" smd custom (at -1.765 0) (size 0.5 2.5) (layers "F.Cu") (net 4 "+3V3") (options (clearance outline) (anchor rect)) (primitives))
  (pad "2" smd custom (at 1.765 0) (size 0.5 2.5) (layers "F.Cu") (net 2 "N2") (options (clearance outline) (anchor rect)) (primitives)))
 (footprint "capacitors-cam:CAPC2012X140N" (layer "F.Cu") (at 108.4 71.5)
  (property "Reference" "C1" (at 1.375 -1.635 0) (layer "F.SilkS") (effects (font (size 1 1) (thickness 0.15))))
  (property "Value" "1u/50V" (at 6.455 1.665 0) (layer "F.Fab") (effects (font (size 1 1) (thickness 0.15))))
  (fp_line (start 0 -0.55) (end 0 0.55) (stroke (width 0.2) (type solid)) (layer "F.SilkS"))
  (pad "1" smd rect (at -0.9 0) (size 1.15 1.45) (layers "F.Cu" "F.Mask" "F.Paste") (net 3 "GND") (solder_mask_margin 0.102))
  (pad "2" smd rect (at 0.9 0) (size 1.15 1.45) (layers "F.Cu" "F.Mask" "F.Paste") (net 11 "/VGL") (solder_mask_margin 0.102)))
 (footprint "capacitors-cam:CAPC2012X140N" (layer "F.Cu") (at 108.55 74.085)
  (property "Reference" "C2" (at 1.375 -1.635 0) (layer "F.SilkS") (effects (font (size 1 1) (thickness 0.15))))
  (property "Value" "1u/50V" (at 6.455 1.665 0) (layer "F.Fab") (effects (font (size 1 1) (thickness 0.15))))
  (fp_line (start 0 -0.55) (end 0 0.55) (stroke (width 0.2) (type solid)) (layer "F.SilkS"))
  (pad "1" smd rect (at -0.9 0) (size 1.15 1.45) (layers "F.Cu" "F.Mask" "F.Paste") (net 3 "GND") (solder_mask_margin 0.102))
  (pad "2" smd rect (at 0.9 0) (size 1.15 1.45) (layers "F.Cu" "F.Mask" "F.Paste") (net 12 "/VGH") (solder_mask_margin 0.102)))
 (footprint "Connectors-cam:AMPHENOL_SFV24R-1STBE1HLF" (layer "F.Cu") (at 73 85 -90)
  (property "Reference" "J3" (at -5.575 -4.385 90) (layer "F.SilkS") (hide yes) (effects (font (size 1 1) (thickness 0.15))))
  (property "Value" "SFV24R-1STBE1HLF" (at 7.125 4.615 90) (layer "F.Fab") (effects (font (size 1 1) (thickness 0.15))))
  (fp_line (start -8.75 2.1) (end 8.75 2.1) (stroke (width 0.127) (type solid)) (layer "F.SilkS"))
  (fp_line (start 8.75 2.1) (end 8.75 0.7) (stroke (width 0.127) (type solid)) (layer "F.SilkS"))
  (fp_line (start -8.75 0.7) (end -8.75 2.1) (stroke (width 0.127) (type solid)) (layer "F.SilkS"))
  (fp_line (start -7.95 0.7) (end -8.75 0.7) (stroke (width 0.127) (type solid)) (layer "F.SilkS"))
  (fp_line (start 7.95 0.7) (end 7.95 -0.38) (stroke (width 0.127) (type solid)) (layer "F.SilkS"))
  (fp_line (start 8.75 0.7) (end 7.95 0.7) (stroke (width 0.127) (type solid)) (layer "F.SilkS"))
  (fp_line (start -7.95 -0.38) (end -7.95 0.7) (stroke (width 0.127) (type solid)) (layer "F.SilkS"))
  (fp_circle (center -5.75 -3.6) (end -5.65 -3.6) (stroke (width 0.2) (type solid)) (fill no) (layer "F.SilkS"))
  (pad "1" smd rect (at -5.75 -2.4 270) (size 0.3 1.4) (layers "F.Cu" "F.Mask" "F.Paste") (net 8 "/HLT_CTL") (solder_mask_margin 0.102))
  (pad "2" smd rect (at -5.25 -2.4 270) (size 0.3 1.4) (layers "F.Cu" "F.Mask" "F.Paste") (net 9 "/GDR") (solder_mask_margin 0.102))
  (pad "3" smd rect (at -4.75 -2.4 270) (size 0.3 1.4) (layers "F.Cu" "F.Mask" "F.Paste") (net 10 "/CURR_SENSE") (solder_mask_margin 0.102))
  (pad "4" smd rect (at -4.25 -2.4 270) (size 0.3 1.4) (layers "F.Cu" "F.Mask" "F.Paste") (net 11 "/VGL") (solder_mask_margin 0.102))
  (pad "5" smd rect (at -3.75 -2.4 270) (size 0.3 1.4) (layers "F.Cu" "F.Mask" "F.Paste") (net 12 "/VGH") (solder_mask_margin 0.102))
  (pad "6" smd rect (at -3.25 -2.4 270) (size 0.3 1.4) (layers "F.Cu" "F.Mask" "F.Paste") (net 13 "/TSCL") (solder_mask_margin 0.102))
  (pad "7" smd rect (at -2.75 -2.4 270) (size 0.3 1.4) (layers "F.Cu" "F.Mask" "F.Paste") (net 14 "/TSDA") (solder_mask_margin 0.102))
  (pad "8" smd rect (at -2.25 -2.4 270) (size 0.3 1.4) (layers "F.Cu" "F.Mask" "F.Paste") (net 15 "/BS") (solder_mask_margin 0.102))
  (pad "9" smd rect (at -1.75 -2.4 270) (size 0.3 1.4) (layers "F.Cu" "F.Mask" "F.Paste") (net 16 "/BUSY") (solder_mask_margin 0.102))
  (pad "10" smd rect (at -1.25 -2.4 270) (size 0.3 1.4) (layers "F.Cu" "F.Mask" "F.Paste") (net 17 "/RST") (solder_mask_margin 0.102))
  (pad "11" smd rect (at -0.75 -2.4 270) (size 0.3 1.4) (layers "F.Cu" "F.Mask" "F.Paste") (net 18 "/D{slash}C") (solder_mask_margin 0.102))
  (pad "12" smd rect (at -0.25 -2.4 270) (size 0.3 1.4) (layers "F.Cu" "F.Mask" "F.Paste") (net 19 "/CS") (solder_mask_margin 0.102))
  (pad "13" smd rect (at 0.25 -2.4 270) (size 0.3 1.4) (layers "F.Cu" "F.Mask" "F.Paste") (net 20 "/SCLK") (solder_mask_margin 0.102))
  (pad "14" smd rect (at 0.75 -2.4 270) (size 0.3 1.4) (layers "F.Cu" "F.Mask" "F.Paste") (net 21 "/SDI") (solder_mask_margin 0.102))
  (pad "15" smd rect (at 1.25 -2.4 270) (size 0.3 1.4) (layers "F.Cu" "F.Mask" "F.Paste") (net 4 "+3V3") (solder_mask_margin 0.102))
  (pad "16" smd rect (at 1.75 -2.4 270) (size 0.3 1.4) (layers "F.Cu" "F.Mask" "F.Paste") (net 4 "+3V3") (solder_mask_margin 0.102))
  (pad "17" smd rect (at 2.25 -2.4 270) (size 0.3 1.4) (layers "F.Cu" "F.Mask" "F.Paste") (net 3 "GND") (solder_mask_margin 0.102))
  (pad "18" smd rect (at 2.75 -2.4 270) (size 0.3 1.4) (layers "F.Cu" "F.Mask" "F.Paste") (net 22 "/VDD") (solder_mask_margin 0.102))
  (pad "19" smd rect (at 3.25 -2.4 270) (size 0.3 1.4) (layers "F.Cu" "F.Mask" "F.Paste") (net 23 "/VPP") (solder_mask_margin 0.102))
  (pad "20" smd rect (at 3.75 -2.4 270) (size 0.3 1.4) (layers "F.Cu" "F.Mask" "F.Paste") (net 24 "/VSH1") (solder_mask_margin 0.102))
  (pad "21" smd rect (at 4.25 -2.4 270) (size 0.3 1.4) (layers "F.Cu" "F.Mask" "F.Paste") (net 1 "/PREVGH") (solder_mask_margin 0.102))
  (pad "22" smd rect (at 4.75 -2.4 270) (size 0.3 1.4) (layers "F.Cu" "F.Mask" "F.Paste") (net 25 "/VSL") (solder_mask_margin 0.102))
  (pad "23" smd rect (at 5.25 -2.4 270) (size 0.3 1.4) (layers "F.Cu" "F.Mask" "F.Paste") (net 7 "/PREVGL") (solder_mask_margin 0.102))
  (pad "24" smd rect (at 5.75 -2.4 270) (size 0.3 1.4) (layers "F.Cu" "F.Mask" "F.Paste") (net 5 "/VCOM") (solder_mask_margin 0.102))
  (pad "SH1" smd custom (at -7.175 -1.5 270) (size 1 1) (layers "F.Cu") (options (clearance outline) (anchor rect)) (primitives))
  (pad "SH2" smd custom (at 7.175 -1.5 270) (size 1 1) (layers "F.Cu") (options (clearance outline) (anchor rect)) (primitives)))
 (gr_poly (pts (xy 100.5 65) (xy 65 65) (xy 65 105) (xy 100.5 105)) (stroke (width 0.05) (type solid)) (fill no) (layer "Edge.Cuts"))
 (segment (start 75.451 79.75) (end 75.5 79.799) (width 0.2) (layer "F.Cu") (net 9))
 (segment (start 75.4 79.75) (end 75.451 79.75) (width 0.2) (layer "F.Cu") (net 9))
 (segment (start 76.401 84.349) (end 76.401 84.299) (width 0.2) (layer "F.Cu") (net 18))
 (segment (start 76.401 84.299) (end 75.449 84.299) (width 0.2) (layer "F.Cu") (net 18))
 (segment (start 75.449 84.299) (end 75.4 84.25) (width 0.2) (layer "F.Cu") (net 18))
 (segment (start 75.449 83.201) (end 75.4 83.25) (width 0.2) (layer "F.Cu") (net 16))
 (segment (start 76.401 83.151) (end 76.401 83.201) (width 0.2) (layer "F.Cu") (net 16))
 (segment (start 76.401 83.201) (end 75.449 83.201) (width 0.2) (layer "F.Cu") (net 16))
 (segment (start 94.16 93.5) (end 95.54 92.12) (width 0.2) (layer "B.Cu") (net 22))
 (segment (start 75.49009 79.25) (end 75.53909 79.299) (width 0.2) (layer "F.Cu") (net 8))
 (segment (start 75.4 79.25) (end 75.49009 79.25) (width 0.2) (layer "F.Cu") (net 8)))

